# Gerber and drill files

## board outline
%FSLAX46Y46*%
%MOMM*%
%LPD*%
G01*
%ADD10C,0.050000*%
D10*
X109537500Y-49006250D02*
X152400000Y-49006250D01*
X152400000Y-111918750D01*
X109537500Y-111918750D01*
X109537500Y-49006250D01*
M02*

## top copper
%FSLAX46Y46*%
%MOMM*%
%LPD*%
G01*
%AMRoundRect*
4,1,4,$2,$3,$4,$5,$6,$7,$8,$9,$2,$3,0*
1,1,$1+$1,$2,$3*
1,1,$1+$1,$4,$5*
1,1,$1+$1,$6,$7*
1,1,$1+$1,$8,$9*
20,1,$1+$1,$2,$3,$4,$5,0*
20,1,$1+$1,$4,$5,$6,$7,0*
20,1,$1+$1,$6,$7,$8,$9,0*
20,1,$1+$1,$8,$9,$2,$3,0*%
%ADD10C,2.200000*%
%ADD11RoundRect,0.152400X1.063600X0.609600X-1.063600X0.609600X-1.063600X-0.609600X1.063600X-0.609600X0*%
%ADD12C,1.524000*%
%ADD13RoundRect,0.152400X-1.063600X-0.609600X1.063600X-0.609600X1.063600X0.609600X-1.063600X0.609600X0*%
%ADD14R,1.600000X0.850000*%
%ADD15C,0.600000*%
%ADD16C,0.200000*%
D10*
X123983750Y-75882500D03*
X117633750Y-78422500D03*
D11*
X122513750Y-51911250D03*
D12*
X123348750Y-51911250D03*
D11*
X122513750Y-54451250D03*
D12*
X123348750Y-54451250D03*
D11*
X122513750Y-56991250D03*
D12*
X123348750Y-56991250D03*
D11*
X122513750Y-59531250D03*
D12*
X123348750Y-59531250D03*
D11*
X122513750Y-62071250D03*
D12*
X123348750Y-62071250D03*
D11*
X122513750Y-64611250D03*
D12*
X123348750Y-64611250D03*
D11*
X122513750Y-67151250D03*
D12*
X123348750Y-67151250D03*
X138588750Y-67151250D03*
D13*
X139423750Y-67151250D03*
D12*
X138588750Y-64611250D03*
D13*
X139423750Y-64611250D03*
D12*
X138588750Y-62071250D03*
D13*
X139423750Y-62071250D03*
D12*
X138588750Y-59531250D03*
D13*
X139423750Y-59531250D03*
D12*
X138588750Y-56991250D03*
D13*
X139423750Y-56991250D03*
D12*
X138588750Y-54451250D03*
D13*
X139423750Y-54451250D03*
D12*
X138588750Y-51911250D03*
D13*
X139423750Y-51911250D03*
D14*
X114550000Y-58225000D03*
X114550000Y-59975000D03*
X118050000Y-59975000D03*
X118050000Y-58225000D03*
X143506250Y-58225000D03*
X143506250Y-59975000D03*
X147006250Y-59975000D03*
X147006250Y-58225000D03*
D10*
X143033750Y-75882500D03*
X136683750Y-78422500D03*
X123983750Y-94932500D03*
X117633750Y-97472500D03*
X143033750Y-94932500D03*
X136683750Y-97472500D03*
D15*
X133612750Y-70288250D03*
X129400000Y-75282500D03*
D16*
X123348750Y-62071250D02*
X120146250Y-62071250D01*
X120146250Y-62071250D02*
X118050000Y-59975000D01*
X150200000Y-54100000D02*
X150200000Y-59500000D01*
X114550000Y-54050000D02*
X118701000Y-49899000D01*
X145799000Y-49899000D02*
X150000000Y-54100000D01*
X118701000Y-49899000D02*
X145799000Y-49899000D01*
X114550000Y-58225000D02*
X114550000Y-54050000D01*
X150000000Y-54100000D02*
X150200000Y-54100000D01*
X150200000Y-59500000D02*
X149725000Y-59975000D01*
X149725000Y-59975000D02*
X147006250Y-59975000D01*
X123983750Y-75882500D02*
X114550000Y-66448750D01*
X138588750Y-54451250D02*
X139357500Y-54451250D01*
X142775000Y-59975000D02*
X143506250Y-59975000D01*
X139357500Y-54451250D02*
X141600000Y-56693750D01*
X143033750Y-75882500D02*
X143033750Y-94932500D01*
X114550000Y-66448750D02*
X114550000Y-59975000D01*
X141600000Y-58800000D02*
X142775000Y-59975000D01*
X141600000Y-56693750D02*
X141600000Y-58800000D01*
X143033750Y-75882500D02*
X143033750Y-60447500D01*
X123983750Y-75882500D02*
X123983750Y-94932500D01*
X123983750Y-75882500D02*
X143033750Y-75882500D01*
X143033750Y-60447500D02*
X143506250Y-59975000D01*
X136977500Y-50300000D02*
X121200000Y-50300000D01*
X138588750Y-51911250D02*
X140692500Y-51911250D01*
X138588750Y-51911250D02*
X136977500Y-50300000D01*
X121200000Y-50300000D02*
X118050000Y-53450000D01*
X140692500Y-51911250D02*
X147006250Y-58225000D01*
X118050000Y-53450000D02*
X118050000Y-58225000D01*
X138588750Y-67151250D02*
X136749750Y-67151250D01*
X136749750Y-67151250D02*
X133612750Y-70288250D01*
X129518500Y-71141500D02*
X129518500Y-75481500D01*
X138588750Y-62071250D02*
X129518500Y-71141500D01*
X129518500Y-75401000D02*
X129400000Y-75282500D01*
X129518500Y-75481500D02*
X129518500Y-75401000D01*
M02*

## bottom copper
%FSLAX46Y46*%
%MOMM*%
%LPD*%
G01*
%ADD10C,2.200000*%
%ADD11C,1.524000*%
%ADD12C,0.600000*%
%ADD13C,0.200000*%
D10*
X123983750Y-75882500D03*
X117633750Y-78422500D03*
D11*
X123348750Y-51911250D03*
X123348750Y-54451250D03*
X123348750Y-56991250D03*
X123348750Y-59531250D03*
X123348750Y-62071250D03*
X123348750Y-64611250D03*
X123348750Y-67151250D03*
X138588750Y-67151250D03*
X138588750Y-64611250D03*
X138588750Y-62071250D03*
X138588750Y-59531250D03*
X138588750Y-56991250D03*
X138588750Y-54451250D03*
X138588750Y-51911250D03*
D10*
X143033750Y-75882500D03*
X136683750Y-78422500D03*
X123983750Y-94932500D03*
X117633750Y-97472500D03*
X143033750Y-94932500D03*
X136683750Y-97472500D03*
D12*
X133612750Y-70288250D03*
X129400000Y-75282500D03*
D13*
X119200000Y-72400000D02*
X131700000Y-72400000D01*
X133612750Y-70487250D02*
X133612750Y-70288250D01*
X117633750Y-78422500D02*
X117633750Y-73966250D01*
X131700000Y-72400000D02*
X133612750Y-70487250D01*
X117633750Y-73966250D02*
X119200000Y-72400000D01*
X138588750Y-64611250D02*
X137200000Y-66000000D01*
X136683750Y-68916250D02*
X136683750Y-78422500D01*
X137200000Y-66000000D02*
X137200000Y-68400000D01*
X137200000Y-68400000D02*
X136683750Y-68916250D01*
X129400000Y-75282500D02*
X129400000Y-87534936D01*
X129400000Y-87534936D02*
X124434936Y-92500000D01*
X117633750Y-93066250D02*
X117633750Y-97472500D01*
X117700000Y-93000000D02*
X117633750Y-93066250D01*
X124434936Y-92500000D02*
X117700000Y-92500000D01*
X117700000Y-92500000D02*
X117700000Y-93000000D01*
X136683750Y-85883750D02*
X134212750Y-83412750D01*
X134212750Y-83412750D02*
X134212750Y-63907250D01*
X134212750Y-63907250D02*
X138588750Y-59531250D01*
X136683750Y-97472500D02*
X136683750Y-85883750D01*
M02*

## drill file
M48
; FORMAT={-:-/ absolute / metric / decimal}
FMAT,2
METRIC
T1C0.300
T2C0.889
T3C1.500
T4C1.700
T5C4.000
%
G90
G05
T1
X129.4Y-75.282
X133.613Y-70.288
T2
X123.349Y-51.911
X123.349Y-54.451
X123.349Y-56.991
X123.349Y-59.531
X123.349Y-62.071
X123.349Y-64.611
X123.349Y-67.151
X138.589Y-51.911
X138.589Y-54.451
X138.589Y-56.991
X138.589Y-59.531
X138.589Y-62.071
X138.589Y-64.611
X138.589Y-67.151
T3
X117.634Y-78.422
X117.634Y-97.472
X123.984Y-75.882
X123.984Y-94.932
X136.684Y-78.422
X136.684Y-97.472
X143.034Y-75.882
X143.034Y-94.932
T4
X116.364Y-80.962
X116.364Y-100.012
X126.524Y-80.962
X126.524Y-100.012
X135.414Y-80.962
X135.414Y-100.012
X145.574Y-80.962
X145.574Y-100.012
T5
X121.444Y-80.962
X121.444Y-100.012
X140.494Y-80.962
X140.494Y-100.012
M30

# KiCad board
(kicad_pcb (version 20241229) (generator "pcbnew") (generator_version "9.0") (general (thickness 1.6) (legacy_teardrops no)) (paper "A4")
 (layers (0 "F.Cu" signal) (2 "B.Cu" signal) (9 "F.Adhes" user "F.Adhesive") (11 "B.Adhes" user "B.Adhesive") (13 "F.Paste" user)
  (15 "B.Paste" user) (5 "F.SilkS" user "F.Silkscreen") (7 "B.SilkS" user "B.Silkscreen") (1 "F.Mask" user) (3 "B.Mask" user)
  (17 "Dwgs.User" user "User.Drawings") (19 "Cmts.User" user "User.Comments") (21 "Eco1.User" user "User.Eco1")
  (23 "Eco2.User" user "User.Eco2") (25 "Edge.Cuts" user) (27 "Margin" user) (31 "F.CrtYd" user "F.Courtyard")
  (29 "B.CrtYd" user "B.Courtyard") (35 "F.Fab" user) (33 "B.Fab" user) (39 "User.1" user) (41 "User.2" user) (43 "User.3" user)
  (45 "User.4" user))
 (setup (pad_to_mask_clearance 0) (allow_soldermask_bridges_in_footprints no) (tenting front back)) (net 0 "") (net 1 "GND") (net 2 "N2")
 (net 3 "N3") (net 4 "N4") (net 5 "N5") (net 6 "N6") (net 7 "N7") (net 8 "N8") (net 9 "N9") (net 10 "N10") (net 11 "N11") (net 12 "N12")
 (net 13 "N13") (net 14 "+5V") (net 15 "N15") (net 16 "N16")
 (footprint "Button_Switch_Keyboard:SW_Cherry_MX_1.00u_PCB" (layer "F.Cu") (at 123.98375 75.8825)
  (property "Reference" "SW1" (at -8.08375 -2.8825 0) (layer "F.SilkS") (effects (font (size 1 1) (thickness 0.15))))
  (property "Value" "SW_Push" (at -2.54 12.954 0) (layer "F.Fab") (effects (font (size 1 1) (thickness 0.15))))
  (pad "" np_thru_hole circle (at -7.62 5.08) (size 1.7 1.7) (drill 1.7) (layers "*.Cu" "*.Mask"))
  (pad "" np_thru_hole circle (at -2.54 5.08) (size 4 4) (drill 4) (layers "*.Cu" "*.Mask"))
  (pad "" np_thru_hole circle (at 2.54 5.08) (size 1.7 1.7) (drill 1.7) (layers "*.Cu" "*.Mask"))
  (pad "1" thru_hole circle (at 0 0) (size 2.2 2.2) (drill 1.5) (layers "*.Cu" "*.Mask") (remove_unused_layers no) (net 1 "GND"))
  (pad "2" thru_hole circle (at -6.35 2.54) (size 2.2 2.2) (drill 1.5) (layers "*.Cu" "*.Mask") (remove_unused_layers no) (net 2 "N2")))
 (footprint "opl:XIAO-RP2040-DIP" (layer "F.Cu") (at 130.96875 59.53125)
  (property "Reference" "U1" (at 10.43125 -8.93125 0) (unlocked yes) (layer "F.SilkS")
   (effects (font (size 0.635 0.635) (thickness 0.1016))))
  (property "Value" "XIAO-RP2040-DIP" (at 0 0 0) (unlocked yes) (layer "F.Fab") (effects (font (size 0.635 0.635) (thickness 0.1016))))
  (pad "1" smd roundrect (at -8.455 -7.62 180) (size 2.432 1.524) (layers "F.Cu" "F.Mask") (roundrect_rratio 0.1) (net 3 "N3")
   (thermal_bridge_angle 45))
  (pad "1" thru_hole circle (at -7.62 -7.62 180) (size 1.524 1.524) (drill 0.889) (layers "*.Cu" "*.Mask") (remove_unused_layers no)
   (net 3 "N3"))
  (pad "2" smd roundrect (at -8.455 -5.08 180) (size 2.432 1.524) (layers "F.Cu" "F.Mask") (roundrect_rratio 0.1) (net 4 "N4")
   (thermal_bridge_angle 45))
  (pad "2" thru_hole circle (at -7.62 -5.08 180) (size 1.524 1.524) (drill 0.889) (layers "*.Cu" "*.Mask") (remove_unused_layers no)
   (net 4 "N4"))
  (pad "3" smd roundrect (at -8.455 -2.54 180) (size 2.432 1.524) (layers "F.Cu" "F.Mask") (roundrect_rratio 0.1) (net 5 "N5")
   (thermal_bridge_angle 45))
  (pad "3" thru_hole circle (at -7.62 -2.54 180) (size 1.524 1.524) (drill 0.889) (layers "*.Cu" "*.Mask") (remove_unused_layers no)
   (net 5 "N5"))
  (pad "4" smd roundrect (at -8.455 0 180) (size 2.432 1.524) (layers "F.Cu" "F.Mask") (roundrect_rratio 0.1) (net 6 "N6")
   (thermal_bridge_angle 45))
  (pad "4" thru_hole circle (at -7.62 0 180) (size 1.524 1.524) (drill 0.889) (layers "*.Cu" "*.Mask") (remove_unused_layers no)
   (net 6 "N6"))
  (pad "5" smd roundrect (at -8.455 2.54 180) (size 2.432 1.524) (layers "F.Cu" "F.Mask") (roundrect_rratio 0.1) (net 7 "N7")
   (thermal_bridge_angle 45))
  (pad "5" thru_hole circle (at -7.62 2.54 180) (size 1.524 1.524) (drill 0.889) (layers "*.Cu" "*.Mask") (remove_unused_layers no)
   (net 7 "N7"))
  (pad "6" smd roundrect (at -8.455 5.08 180) (size 2.432 1.524) (layers "F.Cu" "F.Mask") (roundrect_rratio 0.1) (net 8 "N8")
   (thermal_bridge_angle 45))
  (pad "6" thru_hole circle (at -7.62 5.08 180) (size 1.524 1.524) (drill 0.889) (layers "*.Cu" "*.Mask") (remove_unused_layers no)
   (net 8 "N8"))
  (pad "7" smd roundrect (at -8.455 7.62 180) (size 2.432 1.524) (layers "F.Cu" "F.Mask") (roundrect_rratio 0.1) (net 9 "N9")
   (thermal_bridge_angle 45))
  (pad "7" thru_hole circle (at -7.62 7.62 180) (size 1.524 1.524) (drill 0.889) (layers "*.Cu" "*.Mask") (remove_unused_layers no)
   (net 9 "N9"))
  (pad "8" thru_hole circle (at 7.62 7.62) (size 1.524 1.524) (drill 0.889) (layers "*.Cu" "*.Mask") (remove_unused_layers no) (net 2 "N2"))
  (pad "8" smd roundrect (at 8.455 7.62) (size 2.432 1.524) (layers "F.Cu" "F.Mask") (roundrect_rratio 0.1) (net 2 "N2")
   (thermal_bridge_angle 45))
  (pad "9" thru_hole circle (at 7.62 5.08) (size 1.524 1.524) (drill 0.889) (layers "*.Cu" "*.Mask") (remove_unused_layers no)
   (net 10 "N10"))
  (pad "9" smd roundrect (at 8.455 5.08) (size 2.432 1.524) (layers "F.Cu" "F.Mask") (roundrect_rratio 0.1) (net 10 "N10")
   (thermal_bridge_angle 45))
  (pad "10" thru_hole circle (at 7.62 2.54) (size 1.524 1.524) (drill 0.889) (layers "*.Cu" "*.Mask") (remove_unused_layers no)
   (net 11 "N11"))
  (pad "10" smd roundrect (at 8.455 2.54) (size 2.432 1.524) (layers "F.Cu" "F.Mask") (roundrect_rratio 0.1) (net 11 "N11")
   (thermal_bridge_angle 45))
  (pad "11" thru_hole circle (at 7.62 0) (size 1.524 1.524) (drill 0.889) (layers "*.Cu" "*.Mask") (remove_unused_layers no) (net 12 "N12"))
  (pad "11" smd roundrect (at 8.455 0) (size 2.432 1.524) (layers "F.Cu" "F.Mask") (roundrect_rratio 0.1) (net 12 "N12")
   (thermal_bridge_angle 45))
  (pad "12" thru_hole circle (at 7.62 -2.54) (size 1.524 1.524) (drill 0.889) (layers "*.Cu" "*.Mask") (remove_unused_layers no)
   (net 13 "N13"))
  (pad "12" smd roundrect (at 8.455 -2.54) (size 2.432 1.524) (layers "F.Cu" "F.Mask") (roundrect_rratio 0.1) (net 13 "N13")
   (thermal_bridge_angle 45))
  (pad "13" thru_hole circle (at 7.62 -5.08) (size 1.524 1.524) (drill 0.889) (layers "*.Cu" "*.Mask") (remove_unused_layers no)
   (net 1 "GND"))
  (pad "13" smd roundrect (at 8.455 -5.08) (size 2.432 1.524) (layers "F.Cu" "F.Mask") (roundrect_rratio 0.1) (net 1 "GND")
   (thermal_bridge_angle 45))
  (pad "14" thru_hole circle (at 7.62 -7.62) (size 1.524 1.524) (drill 0.889) (layers "*.Cu" "*.Mask") (remove_unused_layers no)
   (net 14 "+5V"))
  (pad "14" smd roundrect (at 8.455 -7.62) (size 2.432 1.524) (layers "F.Cu" "F.Mask") (roundrect_rratio 0.1) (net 14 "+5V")
   (thermal_bridge_angle 45)))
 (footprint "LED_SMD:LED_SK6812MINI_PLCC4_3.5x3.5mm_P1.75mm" (layer "F.Cu") (at 116.3 59.1)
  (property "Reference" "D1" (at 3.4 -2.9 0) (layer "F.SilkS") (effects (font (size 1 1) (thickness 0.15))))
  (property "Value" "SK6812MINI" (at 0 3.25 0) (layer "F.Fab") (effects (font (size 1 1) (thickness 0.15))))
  (pad "1" smd rect (at -1.75 -0.875) (size 1.6 0.85) (layers "F.Cu" "F.Mask" "F.Paste") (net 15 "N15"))
  (pad "2" smd rect (at -1.75 0.875) (size 1.6 0.85) (layers "F.Cu" "F.Mask" "F.Paste") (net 1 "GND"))
  (pad "3" smd rect (at 1.75 0.875) (size 1.6 0.85) (layers "F.Cu" "F.Mask" "F.Paste") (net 7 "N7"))
  (pad "4" smd rect (at 1.75 -0.875) (size 1.6 0.85) (layers "F.Cu" "F.Mask" "F.Paste") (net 14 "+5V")))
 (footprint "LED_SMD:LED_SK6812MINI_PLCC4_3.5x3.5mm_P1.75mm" (layer "F.Cu") (at 145.25625 59.1)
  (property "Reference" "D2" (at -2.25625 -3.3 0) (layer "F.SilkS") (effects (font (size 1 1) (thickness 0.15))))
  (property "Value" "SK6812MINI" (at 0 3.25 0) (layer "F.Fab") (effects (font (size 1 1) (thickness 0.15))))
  (pad "1" smd rect (at -1.75 -0.875) (size 1.6 0.85) (layers "F.Cu" "F.Mask" "F.Paste") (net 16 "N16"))
  (pad "2" smd rect (at -1.75 0.875) (size 1.6 0.85) (layers "F.Cu" "F.Mask" "F.Paste") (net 1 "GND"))
  (pad "3" smd rect (at 1.75 0.875) (size 1.6 0.85) (layers "F.Cu" "F.Mask" "F.Paste") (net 15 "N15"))
  (pad "4" smd rect (at 1.75 -0.875) (size 1.6 0.85) (layers "F.Cu" "F.Mask" "F.Paste") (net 14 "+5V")))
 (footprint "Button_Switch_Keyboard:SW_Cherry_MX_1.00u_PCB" (layer "F.Cu") (at 143.03375 75.8825)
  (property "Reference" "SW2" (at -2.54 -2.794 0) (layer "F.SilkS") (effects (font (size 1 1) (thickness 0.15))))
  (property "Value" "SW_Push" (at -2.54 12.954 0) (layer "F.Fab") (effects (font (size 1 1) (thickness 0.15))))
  (pad "" np_thru_hole circle (at -7.62 5.08) (size 1.7 1.7) (drill 1.7) (layers "*.Cu" "*.Mask"))
  (pad "" np_thru_hole circle (at -2.54 5.08) (size 4 4) (drill 4) (layers "*.Cu" "*.Mask"))
  (pad "" np_thru_hole circle (at 2.54 5.08) (size 1.7 1.7) (drill 1.7) (layers "*.Cu" "*.Mask"))
  (pad "1" thru_hole circle (at 0 0) (size 2.2 2.2) (drill 1.5) (layers "*.Cu" "*.Mask") (remove_unused_layers no) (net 1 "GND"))
  (pad "2" thru_hole circle (at -6.35 2.54) (size 2.2 2.2) (drill 1.5) (layers "*.Cu" "*.Mask") (remove_unused_layers no) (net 10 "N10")))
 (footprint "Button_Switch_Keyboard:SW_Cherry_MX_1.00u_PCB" (layer "F.Cu") (at 123.98375 94.9325)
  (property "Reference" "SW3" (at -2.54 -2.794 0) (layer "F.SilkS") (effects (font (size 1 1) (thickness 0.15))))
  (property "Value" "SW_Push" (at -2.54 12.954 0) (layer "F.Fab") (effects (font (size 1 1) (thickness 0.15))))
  (pad "" np_thru_hole circle (at -7.62 5.08) (size 1.7 1.7) (drill 1.7) (layers "*.Cu" "*.Mask"))
  (pad "" np_thru_hole circle (at -2.54 5.08) (size 4 4) (drill 4) (layers "*.Cu" "*.Mask"))
  (pad "" np_thru_hole circle (at 2.54 5.08) (size 1.7 1.7) (drill 1.7) (layers "*.Cu" "*.Mask"))
  (pad "1" thru_hole circle (at 0 0) (size 2.2 2.2) (drill 1.5) (layers "*.Cu" "*.Mask") (remove_unused_layers no) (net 1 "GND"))
  (pad "2" thru_hole circle (at -6.35 2.54) (size 2.2 2.2) (drill 1.5) (layers "*.Cu" "*.Mask") (remove_unused_layers no) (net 11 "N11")))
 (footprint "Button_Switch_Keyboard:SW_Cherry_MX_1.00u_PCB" (layer "F.Cu") (at 143.03375 94.9325)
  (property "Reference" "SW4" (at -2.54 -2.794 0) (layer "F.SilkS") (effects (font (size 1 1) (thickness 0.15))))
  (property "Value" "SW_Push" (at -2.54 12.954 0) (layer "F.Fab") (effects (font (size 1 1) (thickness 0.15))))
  (pad "" np_thru_hole circle (at -7.62 5.08) (size 1.7 1.7) (drill 1.7) (layers "*.Cu" "*.Mask"))
  (pad "" np_thru_hole circle (at -2.54 5.08) (size 4 4) (drill 4) (layers "*.Cu" "*.Mask"))
  (pad "" np_thru_hole circle (at 2.54 5.08) (size 1.7 1.7) (drill 1.7) (layers "*.Cu" "*.Mask"))
  (pad "1" thru_hole circle (at 0 0) (size 2.2 2.2) (drill 1.5) (layers "*.Cu" "*.Mask") (remove_unused_layers no) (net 1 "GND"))
  (pad "2" thru_hole circle (at -6.35 2.54) (size 2.2 2.2) (drill 1.5) (layers "*.Cu" "*.Mask") (remove_unused_layers no) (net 12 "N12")))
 (gr_rect (start 109.5375 49.00625) (end 152.4 111.91875) (stroke (width 0.05) (type default)) (fill no) (layer "Edge.Cuts"))
 (segment (start 123.34875 62.07125) (end 120.14625 62.07125) (width 0.2) (layer "F.Cu") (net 7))
 (segment (start 120.14625 62.07125) (end 118.05 59.975) (width 0.2) (layer "F.Cu") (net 7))
 (segment (start 150.2 54.1) (end 150.2 59.5) (width 0.2) (layer "F.Cu") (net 15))
 (segment (start 114.55 54.05) (end 118.701 49.899) (width 0.2) (layer "F.Cu") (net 15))
 (segment (start 145.799 49.899) (end 150 54.1) (width 0.2) (layer "F.Cu") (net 15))
 (segment (start 118.701 49.899) (end 145.799 49.899) (width 0.2) (layer "F.Cu") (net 15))
 (segment (start 114.55 58.225) (end 114.55 54.05) (width 0.2) (layer "F.Cu") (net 15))
 (segment (start 150 54.1) (end 150.2 54.1) (width 0.2) (layer "F.Cu") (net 15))
 (segment (start 150.2 59.5) (end 149.725 59.975) (width 0.2) (layer "F.Cu") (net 15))
 (segment (start 149.725 59.975) (end 147.00625 59.975) (width 0.2) (layer "F.Cu") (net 15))
 (segment (start 123.98375 75.8825) (end 114.55 66.44875) (width 0.2) (layer "F.Cu") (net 1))
 (segment (start 138.58875 54.45125) (end 139.3575 54.45125) (width 0.2) (layer "F.Cu") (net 1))
 (segment (start 142.775 59.975) (end 143.50625 59.975) (width 0.2) (layer "F.Cu") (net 1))
 (segment (start 139.3575 54.45125) (end 141.6 56.69375) (width 0.2) (layer "F.Cu") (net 1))
 (segment (start 143.03375 75.8825) (end 143.03375 94.9325) (width 0.2) (layer "F.Cu") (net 1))
 (segment (start 114.55 66.44875) (end 114.55 59.975) (width 0.2) (layer "F.Cu") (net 1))
 (segment (start 141.6 58.8) (end 142.775 59.975) (width 0.2) (layer "F.Cu") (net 1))
 (segment (start 141.6 56.69375) (end 141.6 58.8) (width 0.2) (layer "F.Cu") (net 1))
 (segment (start 143.03375 75.8825) (end 143.03375 60.4475) (width 0.2) (layer "F.Cu") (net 1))
 (segment (start 123.98375 75.8825) (end 123.98375 94.9325) (width 0.2) (layer "F.Cu") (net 1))
 (segment (start 123.98375 75.8825) (end 143.03375 75.8825) (width 0.2) (layer "F.Cu") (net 1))
 (segment (start 143.03375 60.4475) (end 143.50625 59.975) (width 0.2) (layer "F.Cu") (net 1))
 (segment (start 136.9775 50.3) (end 121.2 50.3) (width 0.2) (layer "F.Cu") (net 14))
 (segment (start 138.58875 51.91125) (end 140.6925 51.91125) (width 0.2) (layer "F.Cu") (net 14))
 (segment (start 138.58875 51.91125) (end 136.9775 50.3) (width 0.2) (layer "F.Cu") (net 14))
 (segment (start 121.2 50.3) (end 118.05 53.45) (width 0.2) (layer "F.Cu") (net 14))
 (segment (start 140.6925 51.91125) (end 147.00625 58.225) (width 0.2) (layer "F.Cu") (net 14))
 (segment (start 118.05 53.45) (end 118.05 58.225) (width 0.2) (layer "F.Cu") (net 14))
 (segment (start 138.58875 67.15125) (end 136.74975 67.15125) (width 0.2) (layer "F.Cu") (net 2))
 (segment (start 136.74975 67.15125) (end 133.61275 70.28825) (width 0.2) (layer "F.Cu") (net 2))
 (via (at 133.61275 70.28825) (size 0.6) (drill 0.3) (layers "F.Cu" "B.Cu") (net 2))
 (segment (start 119.2 72.4) (end 131.7 72.4) (width 0.2) (layer "B.Cu") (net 2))
 (segment (start 133.61275 70.48725) (end 133.61275 70.28825) (width 0.2) (layer "B.Cu") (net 2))
 (segment (start 117.63375 78.4225) (end 117.63375 73.96625) (width 0.2) (layer "B.Cu") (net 2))
 (segment (start 131.7 72.4) (end 133.61275 70.48725) (width 0.2) (layer "B.Cu") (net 2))
 (segment (start 117.63375 73.96625) (end 119.2 72.4) (width 0.2) (layer "B.Cu") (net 2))
 (segment (start 138.58875 64.61125) (end 137.2 66) (width 0.2) (layer "B.Cu") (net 10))
 (segment (start 136.68375 68.91625) (end 136.68375 78.4225) (width 0.2) (layer "B.Cu") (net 10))
 (segment (start 137.2 66) (end 137.2 68.4) (width 0.2) (layer "B.Cu") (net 10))
 (segment (start 137.2 68.4) (end 136.68375 68.91625) (width 0.2) (layer "B.Cu") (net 10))
 (segment (start 129.5185 71.1415) (end 129.5185 75.4815) (width 0.2) (layer "F.Cu") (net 11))
 (segment (start 138.58875 62.07125) (end 129.5185 71.1415) (width 0.2) (layer "F.Cu") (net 11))
 (segment (start 129.5185 75.401) (end 129.4 75.2825) (width 0.2) (layer "F.Cu") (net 11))
 (segment (start 129.5185 75.4815) (end 129.5185 75.401) (width 0.2) (layer "F.Cu") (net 11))
 (via (at 129.4 75.2825) (size 0.6) (drill 0.3) (layers "F.Cu" "B.Cu") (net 11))
 (segment (start 129.4 75.2825) (end 129.4 87.534936) (width 0.2) (layer "B.Cu") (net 11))
 (segment (start 129.4 87.534936) (end 124.434936 92.5) (width 0.2) (layer "B.Cu") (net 11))
 (segment (start 117.63375 93.06625) (end 117.63375 97.4725) (width 0.2) (layer "B.Cu") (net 11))
 (segment (start 117.7 93) (end 117.63375 93.06625) (width 0.2) (layer "B.Cu") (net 11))
 (segment (start 124.434936 92.5) (end 117.7 92.5) (width 0.2) (layer "B.Cu") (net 11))
 (segment (start 117.7 92.5) (end 117.7 93) (width 0.2) (layer "B.Cu") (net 11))
 (segment (start 136.68375 85.88375) (end 134.21275 83.41275) (width 0.2) (layer "B.Cu") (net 12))
 (segment (start 134.21275 83.41275) (end 134.21275 63.90725) (width 0.2) (layer "B.Cu") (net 12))
 (segment (start 134.21275 63.90725) (end 138.58875 59.53125) (width 0.2) (layer "B.Cu") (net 12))
 (segment (start 136.68375 97.4725) (end 136.68375 85.88375) (width 0.2) (layer "B.Cu") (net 12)))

